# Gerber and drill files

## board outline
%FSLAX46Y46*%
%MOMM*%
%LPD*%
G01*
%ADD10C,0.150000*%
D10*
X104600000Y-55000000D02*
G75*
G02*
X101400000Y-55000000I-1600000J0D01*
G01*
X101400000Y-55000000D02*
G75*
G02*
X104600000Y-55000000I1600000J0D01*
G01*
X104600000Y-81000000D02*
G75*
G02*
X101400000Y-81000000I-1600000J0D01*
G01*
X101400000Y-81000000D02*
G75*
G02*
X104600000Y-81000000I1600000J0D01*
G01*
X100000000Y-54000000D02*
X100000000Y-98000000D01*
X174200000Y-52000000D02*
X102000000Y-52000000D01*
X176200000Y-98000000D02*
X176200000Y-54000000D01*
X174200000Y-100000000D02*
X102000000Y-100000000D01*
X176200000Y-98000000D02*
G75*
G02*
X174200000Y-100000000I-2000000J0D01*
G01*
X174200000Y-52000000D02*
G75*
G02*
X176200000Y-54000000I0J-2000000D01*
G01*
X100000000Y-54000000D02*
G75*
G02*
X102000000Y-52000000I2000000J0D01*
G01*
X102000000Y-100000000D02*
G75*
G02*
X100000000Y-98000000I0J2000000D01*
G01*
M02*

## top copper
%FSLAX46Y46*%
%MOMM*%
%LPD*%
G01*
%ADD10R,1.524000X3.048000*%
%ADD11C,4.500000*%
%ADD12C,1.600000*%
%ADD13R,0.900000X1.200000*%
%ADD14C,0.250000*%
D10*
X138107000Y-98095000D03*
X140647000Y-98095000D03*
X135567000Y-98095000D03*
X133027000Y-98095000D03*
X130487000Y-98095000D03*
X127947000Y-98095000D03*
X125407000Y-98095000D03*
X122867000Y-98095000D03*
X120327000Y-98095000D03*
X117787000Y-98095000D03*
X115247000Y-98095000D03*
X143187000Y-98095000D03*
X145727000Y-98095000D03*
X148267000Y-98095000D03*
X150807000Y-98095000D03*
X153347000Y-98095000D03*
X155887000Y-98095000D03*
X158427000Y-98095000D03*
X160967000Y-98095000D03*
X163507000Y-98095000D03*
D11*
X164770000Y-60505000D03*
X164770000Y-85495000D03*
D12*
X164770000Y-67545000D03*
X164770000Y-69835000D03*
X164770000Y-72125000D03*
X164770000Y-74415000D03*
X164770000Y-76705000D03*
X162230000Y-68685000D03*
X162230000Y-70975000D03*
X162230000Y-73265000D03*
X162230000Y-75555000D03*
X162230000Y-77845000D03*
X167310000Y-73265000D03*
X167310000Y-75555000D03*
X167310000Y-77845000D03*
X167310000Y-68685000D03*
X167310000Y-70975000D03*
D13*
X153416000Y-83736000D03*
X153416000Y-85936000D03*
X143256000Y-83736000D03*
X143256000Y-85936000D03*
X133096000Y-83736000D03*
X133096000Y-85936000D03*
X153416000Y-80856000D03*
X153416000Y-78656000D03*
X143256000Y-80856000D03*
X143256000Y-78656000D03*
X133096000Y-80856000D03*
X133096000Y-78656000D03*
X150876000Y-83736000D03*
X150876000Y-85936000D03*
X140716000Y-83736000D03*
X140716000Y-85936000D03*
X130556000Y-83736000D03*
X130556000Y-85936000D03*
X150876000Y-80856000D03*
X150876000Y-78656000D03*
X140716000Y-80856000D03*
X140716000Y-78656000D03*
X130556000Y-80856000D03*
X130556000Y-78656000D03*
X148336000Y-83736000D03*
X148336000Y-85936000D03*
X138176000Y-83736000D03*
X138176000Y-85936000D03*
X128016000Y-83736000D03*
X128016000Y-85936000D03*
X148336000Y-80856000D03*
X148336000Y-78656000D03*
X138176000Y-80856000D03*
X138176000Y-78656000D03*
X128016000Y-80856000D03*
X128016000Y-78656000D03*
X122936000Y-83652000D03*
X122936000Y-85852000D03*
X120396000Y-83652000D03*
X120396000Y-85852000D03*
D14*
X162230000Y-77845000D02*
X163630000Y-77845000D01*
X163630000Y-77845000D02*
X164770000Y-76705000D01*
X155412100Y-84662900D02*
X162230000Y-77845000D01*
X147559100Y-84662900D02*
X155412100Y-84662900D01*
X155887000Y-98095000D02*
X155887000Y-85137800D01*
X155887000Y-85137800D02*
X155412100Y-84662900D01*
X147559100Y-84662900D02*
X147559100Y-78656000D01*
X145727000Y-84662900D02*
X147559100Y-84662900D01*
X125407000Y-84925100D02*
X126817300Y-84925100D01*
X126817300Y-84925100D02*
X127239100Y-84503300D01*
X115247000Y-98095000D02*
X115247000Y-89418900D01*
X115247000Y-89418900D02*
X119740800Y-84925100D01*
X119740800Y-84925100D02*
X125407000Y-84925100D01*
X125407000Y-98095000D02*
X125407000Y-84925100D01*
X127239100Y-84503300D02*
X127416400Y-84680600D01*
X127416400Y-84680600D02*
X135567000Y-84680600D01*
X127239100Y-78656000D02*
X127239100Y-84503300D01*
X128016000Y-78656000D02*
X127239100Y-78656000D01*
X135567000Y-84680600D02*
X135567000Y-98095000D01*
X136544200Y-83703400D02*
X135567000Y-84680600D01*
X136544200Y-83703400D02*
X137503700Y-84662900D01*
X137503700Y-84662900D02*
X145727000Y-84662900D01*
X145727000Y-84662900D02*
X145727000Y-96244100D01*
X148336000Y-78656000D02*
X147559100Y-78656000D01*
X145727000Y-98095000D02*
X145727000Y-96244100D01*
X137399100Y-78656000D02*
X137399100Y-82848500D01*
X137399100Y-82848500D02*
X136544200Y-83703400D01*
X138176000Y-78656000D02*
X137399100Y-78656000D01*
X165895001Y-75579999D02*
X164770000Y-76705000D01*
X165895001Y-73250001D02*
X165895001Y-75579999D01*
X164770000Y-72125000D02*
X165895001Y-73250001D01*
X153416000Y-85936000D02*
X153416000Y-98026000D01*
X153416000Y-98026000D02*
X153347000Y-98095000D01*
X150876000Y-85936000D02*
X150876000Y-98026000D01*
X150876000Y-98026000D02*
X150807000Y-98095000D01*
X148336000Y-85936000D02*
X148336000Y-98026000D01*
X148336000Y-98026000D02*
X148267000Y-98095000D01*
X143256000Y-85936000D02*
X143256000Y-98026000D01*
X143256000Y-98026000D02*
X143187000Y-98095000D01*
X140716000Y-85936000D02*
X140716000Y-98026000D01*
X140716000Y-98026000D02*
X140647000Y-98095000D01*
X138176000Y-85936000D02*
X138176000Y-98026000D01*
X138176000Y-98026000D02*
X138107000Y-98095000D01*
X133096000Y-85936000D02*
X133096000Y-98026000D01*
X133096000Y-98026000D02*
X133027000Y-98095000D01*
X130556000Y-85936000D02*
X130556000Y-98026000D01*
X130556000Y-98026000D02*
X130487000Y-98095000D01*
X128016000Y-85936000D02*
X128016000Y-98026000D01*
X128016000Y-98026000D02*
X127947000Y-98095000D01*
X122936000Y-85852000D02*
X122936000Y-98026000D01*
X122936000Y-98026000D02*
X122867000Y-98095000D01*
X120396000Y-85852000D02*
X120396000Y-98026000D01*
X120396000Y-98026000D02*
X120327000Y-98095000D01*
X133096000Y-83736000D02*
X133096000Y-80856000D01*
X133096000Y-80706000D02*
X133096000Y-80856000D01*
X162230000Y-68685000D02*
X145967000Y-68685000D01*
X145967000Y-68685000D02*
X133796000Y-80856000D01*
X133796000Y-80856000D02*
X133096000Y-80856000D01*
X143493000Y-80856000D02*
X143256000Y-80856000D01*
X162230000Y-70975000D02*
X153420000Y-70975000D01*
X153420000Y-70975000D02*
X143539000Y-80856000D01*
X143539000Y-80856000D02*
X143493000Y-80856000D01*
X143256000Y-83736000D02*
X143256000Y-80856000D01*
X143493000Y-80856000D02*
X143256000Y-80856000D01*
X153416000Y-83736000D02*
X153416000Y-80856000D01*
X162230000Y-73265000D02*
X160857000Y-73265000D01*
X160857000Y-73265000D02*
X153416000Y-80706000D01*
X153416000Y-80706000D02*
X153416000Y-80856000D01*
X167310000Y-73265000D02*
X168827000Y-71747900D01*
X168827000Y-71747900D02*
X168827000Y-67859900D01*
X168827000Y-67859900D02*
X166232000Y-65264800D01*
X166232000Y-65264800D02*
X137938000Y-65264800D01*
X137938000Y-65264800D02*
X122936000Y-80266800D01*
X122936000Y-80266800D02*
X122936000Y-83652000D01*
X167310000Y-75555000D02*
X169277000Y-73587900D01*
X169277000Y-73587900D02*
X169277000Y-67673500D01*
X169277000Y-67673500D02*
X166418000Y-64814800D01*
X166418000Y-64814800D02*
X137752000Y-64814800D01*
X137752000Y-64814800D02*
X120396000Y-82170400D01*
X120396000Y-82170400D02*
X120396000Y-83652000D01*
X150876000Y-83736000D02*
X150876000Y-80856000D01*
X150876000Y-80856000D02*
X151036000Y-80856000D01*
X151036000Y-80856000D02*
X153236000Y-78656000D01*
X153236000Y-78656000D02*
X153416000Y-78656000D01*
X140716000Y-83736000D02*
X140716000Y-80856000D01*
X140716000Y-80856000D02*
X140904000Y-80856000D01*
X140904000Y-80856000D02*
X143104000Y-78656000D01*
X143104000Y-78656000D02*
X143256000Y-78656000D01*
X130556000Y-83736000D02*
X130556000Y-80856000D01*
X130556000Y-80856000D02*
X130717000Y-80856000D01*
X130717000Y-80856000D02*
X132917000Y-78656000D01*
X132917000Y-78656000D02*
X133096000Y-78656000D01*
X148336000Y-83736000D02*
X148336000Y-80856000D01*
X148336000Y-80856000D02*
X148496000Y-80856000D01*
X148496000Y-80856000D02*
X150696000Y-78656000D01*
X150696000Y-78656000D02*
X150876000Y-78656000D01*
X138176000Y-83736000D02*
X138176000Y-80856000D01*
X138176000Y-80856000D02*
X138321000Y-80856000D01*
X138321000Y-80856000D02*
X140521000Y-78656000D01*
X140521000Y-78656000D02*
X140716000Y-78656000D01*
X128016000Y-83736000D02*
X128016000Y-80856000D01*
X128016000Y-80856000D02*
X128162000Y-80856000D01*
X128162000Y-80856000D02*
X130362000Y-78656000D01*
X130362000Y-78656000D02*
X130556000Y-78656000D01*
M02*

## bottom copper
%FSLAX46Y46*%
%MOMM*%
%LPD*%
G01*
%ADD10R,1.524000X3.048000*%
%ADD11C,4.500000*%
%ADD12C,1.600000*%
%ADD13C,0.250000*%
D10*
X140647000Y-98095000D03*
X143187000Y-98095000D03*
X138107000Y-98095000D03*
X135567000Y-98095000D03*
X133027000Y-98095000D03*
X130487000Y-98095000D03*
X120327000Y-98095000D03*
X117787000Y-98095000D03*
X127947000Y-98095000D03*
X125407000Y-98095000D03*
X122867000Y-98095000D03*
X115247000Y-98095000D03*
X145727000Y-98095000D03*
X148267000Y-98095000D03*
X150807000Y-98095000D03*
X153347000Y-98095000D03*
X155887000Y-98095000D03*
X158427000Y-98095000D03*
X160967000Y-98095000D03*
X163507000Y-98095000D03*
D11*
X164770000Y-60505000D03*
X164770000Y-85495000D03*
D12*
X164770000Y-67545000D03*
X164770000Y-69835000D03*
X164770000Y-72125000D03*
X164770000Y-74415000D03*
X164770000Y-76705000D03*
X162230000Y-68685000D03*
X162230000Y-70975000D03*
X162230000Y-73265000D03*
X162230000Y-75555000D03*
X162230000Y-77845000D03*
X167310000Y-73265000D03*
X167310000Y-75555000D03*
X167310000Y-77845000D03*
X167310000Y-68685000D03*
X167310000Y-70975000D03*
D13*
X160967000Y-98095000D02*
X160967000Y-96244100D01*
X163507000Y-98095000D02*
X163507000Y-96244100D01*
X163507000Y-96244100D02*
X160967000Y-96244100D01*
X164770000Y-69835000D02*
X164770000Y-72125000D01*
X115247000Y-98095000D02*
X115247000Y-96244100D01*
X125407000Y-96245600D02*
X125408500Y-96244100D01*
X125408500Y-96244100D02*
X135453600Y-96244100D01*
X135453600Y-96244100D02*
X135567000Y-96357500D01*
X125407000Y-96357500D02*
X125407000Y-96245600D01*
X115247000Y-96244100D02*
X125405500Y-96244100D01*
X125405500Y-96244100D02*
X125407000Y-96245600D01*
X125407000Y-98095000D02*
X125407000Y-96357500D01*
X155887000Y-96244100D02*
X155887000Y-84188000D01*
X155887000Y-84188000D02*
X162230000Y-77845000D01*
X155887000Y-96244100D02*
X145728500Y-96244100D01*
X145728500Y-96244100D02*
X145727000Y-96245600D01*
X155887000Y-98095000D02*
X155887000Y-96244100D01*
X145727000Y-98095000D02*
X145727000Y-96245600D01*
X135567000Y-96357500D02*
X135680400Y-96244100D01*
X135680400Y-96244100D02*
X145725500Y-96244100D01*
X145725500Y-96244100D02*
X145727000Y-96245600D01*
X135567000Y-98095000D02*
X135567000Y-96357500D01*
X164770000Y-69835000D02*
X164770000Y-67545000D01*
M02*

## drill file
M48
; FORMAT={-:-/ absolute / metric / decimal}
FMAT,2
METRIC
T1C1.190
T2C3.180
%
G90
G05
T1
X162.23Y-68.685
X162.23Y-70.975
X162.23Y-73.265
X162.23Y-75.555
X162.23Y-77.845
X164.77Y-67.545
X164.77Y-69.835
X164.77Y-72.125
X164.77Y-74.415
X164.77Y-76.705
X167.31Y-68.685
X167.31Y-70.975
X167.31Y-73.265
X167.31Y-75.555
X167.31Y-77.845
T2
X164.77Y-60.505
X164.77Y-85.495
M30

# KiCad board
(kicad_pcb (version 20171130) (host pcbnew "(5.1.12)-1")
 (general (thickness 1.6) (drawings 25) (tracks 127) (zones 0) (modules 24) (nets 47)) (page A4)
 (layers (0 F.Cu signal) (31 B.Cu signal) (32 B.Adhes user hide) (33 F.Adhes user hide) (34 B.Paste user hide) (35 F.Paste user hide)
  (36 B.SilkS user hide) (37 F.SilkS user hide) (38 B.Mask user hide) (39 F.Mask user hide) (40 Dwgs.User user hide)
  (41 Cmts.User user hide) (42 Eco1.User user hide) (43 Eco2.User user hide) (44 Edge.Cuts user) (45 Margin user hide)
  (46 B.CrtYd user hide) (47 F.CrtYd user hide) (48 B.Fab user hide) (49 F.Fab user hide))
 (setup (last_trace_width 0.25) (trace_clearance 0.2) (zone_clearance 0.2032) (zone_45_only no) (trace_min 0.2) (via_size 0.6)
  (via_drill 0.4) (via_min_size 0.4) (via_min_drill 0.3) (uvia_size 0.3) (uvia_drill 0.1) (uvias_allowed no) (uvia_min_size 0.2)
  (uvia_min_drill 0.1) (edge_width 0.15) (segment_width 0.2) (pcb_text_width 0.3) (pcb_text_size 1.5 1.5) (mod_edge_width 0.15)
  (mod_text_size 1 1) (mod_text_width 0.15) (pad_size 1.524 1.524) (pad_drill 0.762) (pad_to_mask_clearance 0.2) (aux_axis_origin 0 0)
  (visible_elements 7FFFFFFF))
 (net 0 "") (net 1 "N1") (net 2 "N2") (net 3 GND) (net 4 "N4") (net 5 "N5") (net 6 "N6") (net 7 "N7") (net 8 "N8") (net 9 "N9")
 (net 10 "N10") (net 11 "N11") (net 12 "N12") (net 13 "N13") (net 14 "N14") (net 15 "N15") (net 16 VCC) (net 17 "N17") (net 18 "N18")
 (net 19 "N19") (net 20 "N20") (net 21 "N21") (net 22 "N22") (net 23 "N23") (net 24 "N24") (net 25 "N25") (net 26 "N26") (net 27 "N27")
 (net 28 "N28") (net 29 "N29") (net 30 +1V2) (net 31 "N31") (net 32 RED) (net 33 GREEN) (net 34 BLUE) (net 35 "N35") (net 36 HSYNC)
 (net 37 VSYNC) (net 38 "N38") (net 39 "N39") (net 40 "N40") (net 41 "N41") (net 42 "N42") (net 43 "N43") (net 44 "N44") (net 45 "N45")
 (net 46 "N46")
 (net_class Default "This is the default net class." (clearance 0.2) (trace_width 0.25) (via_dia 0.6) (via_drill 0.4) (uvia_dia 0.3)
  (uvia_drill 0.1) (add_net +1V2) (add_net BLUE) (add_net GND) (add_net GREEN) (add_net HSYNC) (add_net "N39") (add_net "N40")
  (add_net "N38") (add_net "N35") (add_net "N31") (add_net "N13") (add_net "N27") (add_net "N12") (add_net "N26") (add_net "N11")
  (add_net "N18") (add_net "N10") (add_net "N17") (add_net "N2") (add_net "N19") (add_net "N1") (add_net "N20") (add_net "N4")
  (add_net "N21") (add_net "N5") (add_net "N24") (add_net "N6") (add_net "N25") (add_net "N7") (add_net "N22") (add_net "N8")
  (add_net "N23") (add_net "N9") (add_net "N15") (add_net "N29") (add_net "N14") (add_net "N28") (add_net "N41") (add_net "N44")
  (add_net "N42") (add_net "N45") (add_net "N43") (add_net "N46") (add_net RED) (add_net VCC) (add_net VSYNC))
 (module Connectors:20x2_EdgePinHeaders (layer F.Cu) (at 139.377 100)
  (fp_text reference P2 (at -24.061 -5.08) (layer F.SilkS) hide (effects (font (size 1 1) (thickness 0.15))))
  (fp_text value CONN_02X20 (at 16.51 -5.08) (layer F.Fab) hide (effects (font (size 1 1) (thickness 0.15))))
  (pad 22 smd rect (at -1.27 -1.905) (size 1.524 3.048) (layers F.Cu F.Paste F.Mask) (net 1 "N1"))
  (pad 20 smd rect (at 1.27 -1.905) (size 1.524 3.048) (layers F.Cu F.Paste F.Mask) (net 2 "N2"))
  (pad 24 smd rect (at -3.81 -1.905) (size 1.524 3.048) (layers F.Cu F.Paste F.Mask) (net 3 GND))
  (pad 26 smd rect (at -6.35 -1.905) (size 1.524 3.048) (layers F.Cu F.Paste F.Mask) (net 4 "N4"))
  (pad 28 smd rect (at -8.89 -1.905) (size 1.524 3.048) (layers F.Cu F.Paste F.Mask) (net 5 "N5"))
  (pad 30 smd rect (at -11.43 -1.905) (size 1.524 3.048) (layers F.Cu F.Paste F.Mask) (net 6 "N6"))
  (pad 32 smd rect (at -13.97 -1.905) (size 1.524 3.048) (layers F.Cu F.Paste F.Mask) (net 3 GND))
  (pad 34 smd rect (at -16.51 -1.905) (size 1.524 3.048) (layers F.Cu F.Paste F.Mask) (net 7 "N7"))
  (pad 36 smd rect (at -19.05 -1.905) (size 1.524 3.048) (layers F.Cu F.Paste F.Mask) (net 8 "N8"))
  (pad 38 smd rect (at -21.59 -1.905) (size 1.524 3.048) (layers F.Cu F.Paste F.Mask) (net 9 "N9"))
  (pad 40 smd rect (at -24.13 -1.905) (size 1.524 3.048) (layers F.Cu F.Paste F.Mask) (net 3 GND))
  (pad 18 smd rect (at 3.81 -1.905) (size 1.524 3.048) (layers F.Cu F.Paste F.Mask) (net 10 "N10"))
  (pad 16 smd rect (at 6.35 -1.905) (size 1.524 3.048) (layers F.Cu F.Paste F.Mask) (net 3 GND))
  (pad 14 smd rect (at 8.89 -1.905) (size 1.524 3.048) (layers F.Cu F.Paste F.Mask) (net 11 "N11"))
  (pad 12 smd rect (at 11.43 -1.905) (size 1.524 3.048) (layers F.Cu F.Paste F.Mask) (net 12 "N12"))
  (pad 10 smd rect (at 13.97 -1.905) (size 1.524 3.048) (layers F.Cu F.Paste F.Mask) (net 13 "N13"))
  (pad 8 smd rect (at 16.51 -1.905) (size 1.524 3.048) (layers F.Cu F.Paste F.Mask) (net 3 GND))
  (pad 6 smd rect (at 19.05 -1.905) (size 1.524 3.048) (layers F.Cu F.Paste F.Mask) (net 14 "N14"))
  (pad 4 smd rect (at 21.59 -1.905) (size 1.524 3.048) (layers F.Cu F.Paste F.Mask) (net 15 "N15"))
  (pad 2 smd rect (at 24.13 -1.905) (size 1.524 3.048) (layers F.Cu F.Paste F.Mask) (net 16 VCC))
  (pad 19 smd rect (at 1.27 -1.905) (size 1.524 3.048) (layers B.Cu B.Paste B.Mask) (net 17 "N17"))
  (pad 17 smd rect (at 3.81 -1.905) (size 1.524 3.048) (layers B.Cu B.Paste B.Mask) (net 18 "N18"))
  (pad 21 smd rect (at -1.27 -1.905) (size 1.524 3.048) (layers B.Cu B.Paste B.Mask) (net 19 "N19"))
  (pad 23 smd rect (at -3.81 -1.905) (size 1.524 3.048) (layers B.Cu B.Paste B.Mask) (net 3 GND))
  (pad 25 smd rect (at -6.35 -1.905) (size 1.524 3.048) (layers B.Cu B.Paste B.Mask) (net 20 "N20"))
  (pad 27 smd rect (at -8.89 -1.905) (size 1.524 3.048) (layers B.Cu B.Paste B.Mask) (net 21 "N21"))
  (pad 35 smd rect (at -19.05 -1.905) (size 1.524 3.048) (layers B.Cu B.Paste B.Mask) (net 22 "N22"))
  (pad 37 smd rect (at -21.59 -1.905) (size 1.524 3.048) (layers B.Cu B.Paste B.Mask) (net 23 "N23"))
  (pad 29 smd rect (at -11.43 -1.905) (size 1.524 3.048) (layers B.Cu B.Paste B.Mask) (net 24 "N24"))
  (pad 31 smd rect (at -13.97 -1.905) (size 1.524 3.048) (layers B.Cu B.Paste B.Mask) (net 3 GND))
  (pad 33 smd rect (at -16.51 -1.905) (size 1.524 3.048) (layers B.Cu B.Paste B.Mask) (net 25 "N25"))
  (pad 39 smd rect (at -24.13 -1.905) (size 1.524 3.048) (layers B.Cu B.Paste B.Mask) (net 3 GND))
  (pad 15 smd rect (at 6.35 -1.905) (size 1.524 3.048) (layers B.Cu B.Paste B.Mask) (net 3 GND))
  (pad 13 smd rect (at 8.89 -1.905) (size 1.524 3.048) (layers B.Cu B.Paste B.Mask) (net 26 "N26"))
  (pad 11 smd rect (at 11.43 -1.905) (size 1.524 3.048) (layers B.Cu B.Paste B.Mask) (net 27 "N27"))
  (pad 9 smd rect (at 13.97 -1.905) (size 1.524 3.048) (layers B.Cu B.Paste B.Mask) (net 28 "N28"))
  (pad 7 smd rect (at 16.51 -1.905) (size 1.524 3.048) (layers B.Cu B.Paste B.Mask) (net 3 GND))
  (pad 5 smd rect (at 19.05 -1.905) (size 1.524 3.048) (layers B.Cu B.Paste B.Mask) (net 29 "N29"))
  (pad 3 smd rect (at 21.59 -1.905) (size 1.524 3.048) (layers B.Cu B.Paste B.Mask) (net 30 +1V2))
  (pad 1 smd rect (at 24.13 -1.905) (size 1.524 3.048) (layers B.Cu B.Paste B.Mask) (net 30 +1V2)))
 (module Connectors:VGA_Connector (layer F.Cu) (at 176.2 73)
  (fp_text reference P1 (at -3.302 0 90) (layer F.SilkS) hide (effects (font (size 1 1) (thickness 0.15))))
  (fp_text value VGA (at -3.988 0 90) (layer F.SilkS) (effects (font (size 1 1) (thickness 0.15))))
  (pad "" thru_hole circle (at -11.43 -12.495) (size 4.5 4.5) (drill 3.18) (layers *.Cu *.Mask F.SilkS))
  (pad "" thru_hole circle (at -11.43 12.495) (size 4.5 4.5) (drill 3.18) (layers *.Cu *.Mask F.SilkS))
  (pad 6 thru_hole circle (at -11.43 -5.455) (size 1.6 1.6) (drill 1.19) (layers *.Cu *.Mask F.SilkS) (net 3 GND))
  (pad 7 thru_hole circle (at -11.43 -3.165) (size 1.6 1.6) (drill 1.19) (layers *.Cu *.Mask F.SilkS) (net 3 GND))
  (pad 8 thru_hole circle (at -11.43 -0.875) (size 1.6 1.6) (drill 1.19) (layers *.Cu *.Mask F.SilkS) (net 3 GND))
  (pad 9 thru_hole circle (at -11.43 1.415) (size 1.6 1.6) (drill 1.19) (layers *.Cu *.Mask F.SilkS) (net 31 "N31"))
  (pad 10 thru_hole circle (at -11.43 3.705) (size 1.6 1.6) (drill 1.19) (layers *.Cu *.Mask F.SilkS) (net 3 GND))
  (pad 1 thru_hole circle (at -13.97 -4.315) (size 1.6 1.6) (drill 1.19) (layers *.Cu *.Mask F.SilkS) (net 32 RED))
  (pad 2 thru_hole circle (at -13.97 -2.025) (size 1.6 1.6) (drill 1.19) (layers *.Cu *.Mask F.SilkS) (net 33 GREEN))
  (pad 3 thru_hole circle (at -13.97 0.265) (size 1.6 1.6) (drill 1.19) (layers *.Cu *.Mask F.SilkS) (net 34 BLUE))
  (pad 4 thru_hole circle (at -13.97 2.555) (size 1.6 1.6) (drill 1.19) (layers *.Cu *.Mask F.SilkS) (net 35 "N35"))
  (pad 5 thru_hole circle (at -13.97 4.845) (size 1.6 1.6) (drill 1.19) (layers *.Cu *.Mask F.SilkS) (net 3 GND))
  (pad 13 thru_hole circle (at -8.89 0.265) (size 1.6 1.6) (drill 1.19) (layers *.Cu *.Mask F.SilkS) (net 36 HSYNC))
  (pad 14 thru_hole circle (at -8.89 2.555) (size 1.6 1.6) (drill 1.19) (layers *.Cu *.Mask F.SilkS) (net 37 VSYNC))
  (pad 15 thru_hole circle (at -8.89 4.845) (size 1.6 1.6) (drill 1.19) (layers *.Cu *.Mask F.SilkS) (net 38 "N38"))
  (pad 11 thru_hole circle (at -8.89 -4.315) (size 1.6 1.6) (drill 1.19) (layers *.Cu *.Mask F.SilkS) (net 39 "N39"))
  (pad 12 thru_hole circle (at -8.89 -2.025) (size 1.6 1.6) (drill 1.19) (layers *.Cu *.Mask F.SilkS) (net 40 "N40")))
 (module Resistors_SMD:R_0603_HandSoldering (layer F.Cu) (at 153.416 84.836 270)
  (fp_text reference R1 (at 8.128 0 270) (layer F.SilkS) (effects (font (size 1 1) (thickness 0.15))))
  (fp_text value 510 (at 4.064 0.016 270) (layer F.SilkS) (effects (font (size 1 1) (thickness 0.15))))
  (pad 1 smd rect (at -1.1 0 270) (size 1.2 0.9) (layers F.Cu F.Paste F.Mask) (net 34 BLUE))
  (pad 2 smd rect (at 1.1 0 270) (size 1.2 0.9) (layers F.Cu F.Paste F.Mask) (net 13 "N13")))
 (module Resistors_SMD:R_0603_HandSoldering (layer F.Cu) (at 143.256 84.836 270)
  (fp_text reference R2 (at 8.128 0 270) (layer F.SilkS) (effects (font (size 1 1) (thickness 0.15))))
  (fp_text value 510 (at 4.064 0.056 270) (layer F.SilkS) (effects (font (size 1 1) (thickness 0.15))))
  (pad 1 smd rect (at -1.1 0 270) (size 1.2 0.9) (layers F.Cu F.Paste F.Mask) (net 33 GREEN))
  (pad 2 smd rect (at 1.1 0 270) (size 1.2 0.9) (layers F.Cu F.Paste F.Mask) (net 10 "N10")))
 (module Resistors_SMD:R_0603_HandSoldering (layer F.Cu) (at 133.096 84.836 270)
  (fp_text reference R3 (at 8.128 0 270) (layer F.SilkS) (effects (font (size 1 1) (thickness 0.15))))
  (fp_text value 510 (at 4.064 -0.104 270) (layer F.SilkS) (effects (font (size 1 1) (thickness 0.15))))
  (pad 1 smd rect (at -1.1 0 270) (size 1.2 0.9) (layers F.Cu F.Paste F.Mask) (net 32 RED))
  (pad 2 smd rect (at 1.1 0 270) (size 1.2 0.9) (layers F.Cu F.Paste F.Mask) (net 4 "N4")))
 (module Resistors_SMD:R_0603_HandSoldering (layer F.Cu) (at 153.416 79.756 90)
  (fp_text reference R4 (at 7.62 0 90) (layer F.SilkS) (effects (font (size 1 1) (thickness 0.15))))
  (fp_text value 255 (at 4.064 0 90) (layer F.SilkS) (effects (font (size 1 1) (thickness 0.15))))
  (pad 1 smd rect (at -1.1 0 90) (size 1.2 0.9) (layers F.Cu F.Paste F.Mask) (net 34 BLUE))
  (pad 2 smd rect (at 1.1 0 90) (size 1.2 0.9) (layers F.Cu F.Paste F.Mask) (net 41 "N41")))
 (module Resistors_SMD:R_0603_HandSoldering (layer F.Cu) (at 143.256 79.756 90)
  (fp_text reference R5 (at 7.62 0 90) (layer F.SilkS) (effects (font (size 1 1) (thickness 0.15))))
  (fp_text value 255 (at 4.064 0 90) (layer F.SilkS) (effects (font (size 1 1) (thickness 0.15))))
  (pad 1 smd rect (at -1.1 0 90) (size 1.2 0.9) (layers F.Cu F.Paste F.Mask) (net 33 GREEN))
  (pad 2 smd rect (at 1.1 0 90) (size 1.2 0.9) (layers F.Cu F.Paste F.Mask) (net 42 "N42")))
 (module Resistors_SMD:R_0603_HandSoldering (layer F.Cu) (at 133.096 79.756 90)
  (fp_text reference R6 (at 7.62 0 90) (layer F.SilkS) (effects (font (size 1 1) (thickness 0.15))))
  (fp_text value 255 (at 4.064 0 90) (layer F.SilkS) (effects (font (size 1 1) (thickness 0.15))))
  (pad 1 smd rect (at -1.1 0 90) (size 1.2 0.9) (layers F.Cu F.Paste F.Mask) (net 32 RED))
  (pad 2 smd rect (at 1.1 0 90) (size 1.2 0.9) (layers F.Cu F.Paste F.Mask) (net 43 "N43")))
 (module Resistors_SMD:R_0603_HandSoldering (layer F.Cu) (at 150.876 84.836 270)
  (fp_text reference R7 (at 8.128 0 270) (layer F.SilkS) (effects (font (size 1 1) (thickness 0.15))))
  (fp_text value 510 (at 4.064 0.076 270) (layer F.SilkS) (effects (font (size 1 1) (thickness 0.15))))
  (pad 1 smd rect (at -1.1 0 270) (size 1.2 0.9) (layers F.Cu F.Paste F.Mask) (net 41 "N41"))
  (pad 2 smd rect (at 1.1 0 270) (size 1.2 0.9) (layers F.Cu F.Paste F.Mask) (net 12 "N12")))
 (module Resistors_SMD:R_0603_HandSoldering (layer F.Cu) (at 140.716 84.836 270)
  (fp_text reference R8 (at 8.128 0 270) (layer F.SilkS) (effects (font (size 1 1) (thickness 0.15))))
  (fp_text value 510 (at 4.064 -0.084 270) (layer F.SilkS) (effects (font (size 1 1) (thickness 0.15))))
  (pad 1 smd rect (at -1.1 0 270) (size 1.2 0.9) (layers F.Cu F.Paste F.Mask) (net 42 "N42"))
  (pad 2 smd rect (at 1.1 0 270) (size 1.2 0.9) (layers F.Cu F.Paste F.Mask) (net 2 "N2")))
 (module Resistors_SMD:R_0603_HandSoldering (layer F.Cu) (at 130.556 84.836 270)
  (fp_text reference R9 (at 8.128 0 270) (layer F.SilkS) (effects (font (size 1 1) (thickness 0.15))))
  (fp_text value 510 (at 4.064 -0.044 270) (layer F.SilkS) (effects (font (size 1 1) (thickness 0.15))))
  (pad 1 smd rect (at -1.1 0 270) (size 1.2 0.9) (layers F.Cu F.Paste F.Mask) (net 43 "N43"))
  (pad 2 smd rect (at 1.1 0 270) (size 1.2 0.9) (layers F.Cu F.Paste F.Mask) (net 5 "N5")))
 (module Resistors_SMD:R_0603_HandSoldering (layer F.Cu) (at 150.876 79.756 90)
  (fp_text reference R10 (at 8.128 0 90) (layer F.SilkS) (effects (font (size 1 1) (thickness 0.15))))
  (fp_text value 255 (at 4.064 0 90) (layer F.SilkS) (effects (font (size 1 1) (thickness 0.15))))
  (pad 1 smd rect (at -1.1 0 90) (size 1.2 0.9) (layers F.Cu F.Paste F.Mask) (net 41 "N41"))
  (pad 2 smd rect (at 1.1 0 90) (size 1.2 0.9) (layers F.Cu F.Paste F.Mask) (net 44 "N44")))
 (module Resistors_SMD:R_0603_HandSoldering (layer F.Cu) (at 140.716 79.756 90)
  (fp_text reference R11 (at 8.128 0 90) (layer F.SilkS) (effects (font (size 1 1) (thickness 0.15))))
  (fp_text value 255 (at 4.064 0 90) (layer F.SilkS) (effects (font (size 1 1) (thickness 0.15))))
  (pad 1 smd rect (at -1.1 0 90) (size 1.2 0.9) (layers F.Cu F.Paste F.Mask) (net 42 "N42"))
  (pad 2 smd rect (at 1.1 0 90) (size 1.2 0.9) (layers F.Cu F.Paste F.Mask) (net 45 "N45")))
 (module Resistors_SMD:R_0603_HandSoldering (layer F.Cu) (at 130.556 79.756 90)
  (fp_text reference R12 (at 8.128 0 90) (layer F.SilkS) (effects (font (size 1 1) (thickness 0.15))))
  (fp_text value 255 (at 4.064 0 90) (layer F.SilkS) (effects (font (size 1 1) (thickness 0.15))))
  (pad 1 smd rect (at -1.1 0 90) (size 1.2 0.9) (layers F.Cu F.Paste F.Mask) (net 43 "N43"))
  (pad 2 smd rect (at 1.1 0 90) (size 1.2 0.9) (layers F.Cu F.Paste F.Mask) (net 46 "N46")))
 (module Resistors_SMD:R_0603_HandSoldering (layer F.Cu) (at 148.336 84.836 270)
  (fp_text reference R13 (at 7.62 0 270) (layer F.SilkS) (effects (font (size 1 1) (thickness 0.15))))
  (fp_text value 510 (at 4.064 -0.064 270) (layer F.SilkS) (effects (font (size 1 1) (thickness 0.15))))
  (pad 1 smd rect (at -1.1 0 270) (size 1.2 0.9) (layers F.Cu F.Paste F.Mask) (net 44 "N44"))
  (pad 2 smd rect (at 1.1 0 270) (size 1.2 0.9) (layers F.Cu F.Paste F.Mask) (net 11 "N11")))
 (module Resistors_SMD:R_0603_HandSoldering (layer F.Cu) (at 138.176 84.836 270)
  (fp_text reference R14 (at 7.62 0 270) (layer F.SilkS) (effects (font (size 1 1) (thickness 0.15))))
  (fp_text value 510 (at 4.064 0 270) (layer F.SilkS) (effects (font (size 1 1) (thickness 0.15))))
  (pad 1 smd rect (at -1.1 0 270) (size 1.2 0.9) (layers F.Cu F.Paste F.Mask) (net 45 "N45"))
  (pad 2 smd rect (at 1.1 0 270) (size 1.2 0.9) (layers F.Cu F.Paste F.Mask) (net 1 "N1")))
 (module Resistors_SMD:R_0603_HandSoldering (layer F.Cu) (at 128.016 84.836 270)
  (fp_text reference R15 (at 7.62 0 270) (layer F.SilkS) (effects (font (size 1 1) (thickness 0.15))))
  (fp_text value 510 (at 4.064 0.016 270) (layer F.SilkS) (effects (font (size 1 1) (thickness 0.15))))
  (pad 1 smd rect (at -1.1 0 270) (size 1.2 0.9) (layers F.Cu F.Paste F.Mask) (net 46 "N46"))
  (pad 2 smd rect (at 1.1 0 270) (size 1.2 0.9) (layers F.Cu F.Paste F.Mask) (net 6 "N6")))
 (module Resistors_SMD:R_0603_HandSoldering (layer F.Cu) (at 148.336 79.756 90)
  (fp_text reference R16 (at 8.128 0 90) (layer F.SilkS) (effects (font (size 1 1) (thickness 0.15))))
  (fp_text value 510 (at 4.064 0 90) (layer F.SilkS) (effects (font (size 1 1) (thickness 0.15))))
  (pad 1 smd rect (at -1.1 0 90) (size 1.2 0.9) (layers F.Cu F.Paste F.Mask) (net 44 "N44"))
  (pad 2 smd rect (at 1.1 0 90) (size 1.2 0.9) (layers F.Cu F.Paste F.Mask) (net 3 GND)))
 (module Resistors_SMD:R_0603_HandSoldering (layer F.Cu) (at 138.176 79.756 90)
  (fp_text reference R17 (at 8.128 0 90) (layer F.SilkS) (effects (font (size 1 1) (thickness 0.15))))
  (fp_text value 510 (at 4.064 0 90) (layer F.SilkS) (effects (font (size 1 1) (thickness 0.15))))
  (pad 1 smd rect (at -1.1 0 90) (size 1.2 0.9) (layers F.Cu F.Paste F.Mask) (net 45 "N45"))
  (pad 2 smd rect (at 1.1 0 90) (size 1.2 0.9) (layers F.Cu F.Paste F.Mask) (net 3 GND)))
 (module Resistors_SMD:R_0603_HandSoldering (layer F.Cu) (at 128.016 79.756 90)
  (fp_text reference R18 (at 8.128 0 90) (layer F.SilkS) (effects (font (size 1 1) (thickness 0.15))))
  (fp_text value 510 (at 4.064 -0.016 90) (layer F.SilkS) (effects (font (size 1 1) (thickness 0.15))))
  (pad 1 smd rect (at -1.1 0 90) (size 1.2 0.9) (layers F.Cu F.Paste F.Mask) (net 46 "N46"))
  (pad 2 smd rect (at 1.1 0 90) (size 1.2 0.9) (layers F.Cu F.Paste F.Mask) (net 3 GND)))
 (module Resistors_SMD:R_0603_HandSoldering (layer F.Cu) (at 122.936 84.752 270)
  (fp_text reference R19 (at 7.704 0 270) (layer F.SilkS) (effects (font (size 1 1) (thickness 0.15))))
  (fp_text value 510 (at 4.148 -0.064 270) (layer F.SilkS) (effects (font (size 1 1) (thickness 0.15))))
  (pad 1 smd rect (at -1.1 0 270) (size 1.2 0.9) (layers F.Cu F.Paste F.Mask) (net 36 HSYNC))
  (pad 2 smd rect (at 1.1 0 270) (size 1.2 0.9) (layers F.Cu F.Paste F.Mask) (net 7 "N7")))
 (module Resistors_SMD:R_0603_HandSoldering (layer F.Cu) (at 120.396 84.752 270)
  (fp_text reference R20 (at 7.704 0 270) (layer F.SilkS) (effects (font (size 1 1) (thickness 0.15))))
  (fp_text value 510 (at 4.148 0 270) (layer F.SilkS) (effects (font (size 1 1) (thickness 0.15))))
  (pad 1 smd rect (at -1.1 0 270) (size 1.2 0.9) (layers F.Cu F.Paste F.Mask) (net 37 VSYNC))
  (pad 2 smd rect (at 1.1 0 270) (size 1.2 0.9) (layers F.Cu F.Paste F.Mask) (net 8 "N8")))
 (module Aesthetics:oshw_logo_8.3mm (layer B.Cu) (at 157.988 90.424 180)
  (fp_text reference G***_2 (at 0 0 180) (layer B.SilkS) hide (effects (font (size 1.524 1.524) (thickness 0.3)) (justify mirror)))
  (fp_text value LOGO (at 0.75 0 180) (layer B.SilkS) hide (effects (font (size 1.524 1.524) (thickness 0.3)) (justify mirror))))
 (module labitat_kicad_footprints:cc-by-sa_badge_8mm (layer B.Cu) (at 124.968 90.424 180)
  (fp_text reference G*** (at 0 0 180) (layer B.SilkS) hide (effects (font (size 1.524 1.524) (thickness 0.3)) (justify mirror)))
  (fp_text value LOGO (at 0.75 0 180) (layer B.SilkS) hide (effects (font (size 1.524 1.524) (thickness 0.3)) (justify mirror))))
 (gr_circle (center 103 55) (end 101.4 55) (layer Edge.Cuts) (width 0.15))
 (gr_circle (center 103 81) (end 101.4 81) (layer Edge.Cuts) (width 0.15))
 (gr_line (start 100 54) (end 100 98) (layer Edge.Cuts) (width 0.15))
 (gr_line (start 174.2 52) (end 102 52) (layer Edge.Cuts) (width 0.15))
 (gr_line (start 176.2 98) (end 176.2 54) (layer Edge.Cuts) (width 0.15))
 (gr_line (start 174.2 100) (end 102 100) (layer Edge.Cuts) (width 0.15))
 (gr_arc (start 174.2 98) (end 176.2 98) (angle 90) (layer Edge.Cuts) (width 0.15))
 (gr_arc (start 174.2 54) (end 174.2 52) (angle 90) (layer Edge.Cuts) (width 0.15))
 (gr_arc (start 102 54) (end 100 54) (angle 90) (layer Edge.Cuts) (width 0.15))
 (gr_arc (start 102 98) (end 102 100) (angle 90) (layer Edge.Cuts) (width 0.15))
 (segment (start 160.967 98.095) (end 160.967 96.2441) (width 0.25) (layer B.Cu) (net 30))
 (segment (start 163.507 98.095) (end 163.507 96.2441) (width 0.25) (layer B.Cu) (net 30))
 (segment (start 163.507 96.2441) (end 160.967 96.2441) (width 0.25) (layer B.Cu) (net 30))
 (segment (start 162.23 77.845) (end 163.63 77.845) (width 0.25) (layer F.Cu) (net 3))
 (segment (start 163.63 77.845) (end 164.77 76.705) (width 0.25) (layer F.Cu) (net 3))
 (segment (start 155.4121 84.6629) (end 162.23 77.845) (width 0.25) (layer F.Cu) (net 3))
 (segment (start 147.5591 84.6629) (end 155.4121 84.6629) (width 0.25) (layer F.Cu) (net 3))
 (segment (start 155.887 98.095) (end 155.887 85.1378) (width 0.25) (layer F.Cu) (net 3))
 (segment (start 155.887 85.1378) (end 155.4121 84.6629) (width 0.25) (layer F.Cu) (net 3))
 (segment (start 147.5591 84.6629) (end 147.5591 78.656) (width 0.25) (layer F.Cu) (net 3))
 (segment (start 145.727 84.6629) (end 147.5591 84.6629) (width 0.25) (layer F.Cu) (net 3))
 (segment (start 164.77 69.835) (end 164.77 72.125) (width 0.25) (layer B.Cu) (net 3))
 (segment (start 125.407 84.9251) (end 126.8173 84.9251) (width 0.25) (layer F.Cu) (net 3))
 (segment (start 126.8173 84.9251) (end 127.2391 84.5033) (width 0.25) (layer F.Cu) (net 3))
 (segment (start 115.247 98.095) (end 115.247 89.4189) (width 0.25) (layer F.Cu) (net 3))
 (segment (start 115.247 89.4189) (end 119.7408 84.9251) (width 0.25) (layer F.Cu) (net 3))
 (segment (start 119.7408 84.9251) (end 125.407 84.9251) (width 0.25) (layer F.Cu) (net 3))
 (segment (start 125.407 98.095) (end 125.407 84.9251) (width 0.25) (layer F.Cu) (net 3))
 (segment (start 127.2391 84.5033) (end 127.4164 84.6806) (width 0.25) (layer F.Cu) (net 3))
 (segment (start 127.4164 84.6806) (end 135.567 84.6806) (width 0.25) (layer F.Cu) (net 3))
 (segment (start 127.2391 78.656) (end 127.2391 84.5033) (width 0.25) (layer F.Cu) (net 3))
 (segment (start 128.016 78.656) (end 127.2391 78.656) (width 0.25) (layer F.Cu) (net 3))
 (segment (start 135.567 84.6806) (end 135.567 98.095) (width 0.25) (layer F.Cu) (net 3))
 (segment (start 136.5442 83.7034) (end 135.567 84.6806) (width 0.25) (layer F.Cu) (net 3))
 (segment (start 115.247 98.095) (end 115.247 96.2441) (width 0.25) (layer B.Cu) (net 3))
 (segment (start 125.407 96.2456) (end 125.4085 96.2441) (width 0.25) (layer B.Cu) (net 3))
 (segment (start 125.4085 96.2441) (end 135.4536 96.2441) (width 0.25) (layer B.Cu) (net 3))
 (segment (start 135.4536 96.2441) (end 135.567 96.3575) (width 0.25) (layer B.Cu) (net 3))
 (segment (start 125.407 96.3575) (end 125.407 96.2456) (width 0.25) (layer B.Cu) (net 3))
 (segment (start 115.247 96.2441) (end 125.4055 96.2441) (width 0.25) (layer B.Cu) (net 3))
 (segment (start 125.4055 96.2441) (end 125.407 96.2456) (width 0.25) (layer B.Cu) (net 3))
 (segment (start 125.407 98.095) (end 125.407 96.3575) (width 0.25) (layer B.Cu) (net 3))
 (segment (start 155.887 96.2441) (end 155.887 84.188) (width 0.25) (layer B.Cu) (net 3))
 (segment (start 155.887 84.188) (end 162.23 77.845) (width 0.25) (layer B.Cu) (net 3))
 (segment (start 155.887 96.2441) (end 145.7285 96.2441) (width 0.25) (layer B.Cu) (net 3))
 (segment (start 145.7285 96.2441) (end 145.727 96.2456) (width 0.25) (layer B.Cu) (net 3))
 (segment (start 155.887 98.095) (end 155.887 96.2441) (width 0.25) (layer B.Cu) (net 3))
 (segment (start 136.5442 83.7034) (end 137.5037 84.6629) (width 0.25) (layer F.Cu) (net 3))
 (segment (start 137.5037 84.6629) (end 145.727 84.6629) (width 0.25) (layer F.Cu) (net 3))
 (segment (start 145.727 84.6629) (end 145.727 96.2441) (width 0.25) (layer F.Cu) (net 3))
 (segment (start 148.336 78.656) (end 147.5591 78.656) (width 0.25) (layer F.Cu) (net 3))
 (segment (start 145.727 98.095) (end 145.727 96.2441) (width 0.25) (layer F.Cu) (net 3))
 (segment (start 145.727 98.095) (end 145.727 96.2456) (width 0.25) (layer B.Cu) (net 3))
 (segment (start 135.567 96.3575) (end 135.6804 96.2441) (width 0.25) (layer B.Cu) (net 3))
 (segment (start 135.6804 96.2441) (end 145.7255 96.2441) (width 0.25) (layer B.Cu) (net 3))
 (segment (start 145.7255 96.2441) (end 145.727 96.2456) (width 0.25) (layer B.Cu) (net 3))
 (segment (start 135.567 98.095) (end 135.567 96.3575) (width 0.25) (layer B.Cu) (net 3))
 (segment (start 137.3991 78.656) (end 137.3991 82.8485) (width 0.25) (layer F.Cu) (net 3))
 (segment (start 137.3991 82.8485) (end 136.5442 83.7034) (width 0.25) (layer F.Cu) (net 3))
 (segment (start 138.176 78.656) (end 137.3991 78.656) (width 0.25) (layer F.Cu) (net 3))
 (segment (start 164.77 69.835) (end 164.77 67.545) (width 0.25) (layer B.Cu) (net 3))
 (segment (start 165.895001 75.579999) (end 164.77 76.705) (width 0.25) (layer F.Cu) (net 3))
 (segment (start 165.895001 73.250001) (end 165.895001 75.579999) (width 0.25) (layer F.Cu) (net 3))
 (segment (start 164.77 72.125) (end 165.895001 73.250001) (width 0.25) (layer F.Cu) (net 3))
 (segment (start 153.416 85.936) (end 153.416 98.026) (width 0.25) (layer F.Cu) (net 13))
 (segment (start 153.416 98.026) (end 153.347 98.095) (width 0.25) (layer F.Cu) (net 13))
 (segment (start 150.876 85.936) (end 150.876 98.026) (width 0.25) (layer F.Cu) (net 12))
 (segment (start 150.876 98.026) (end 150.807 98.095) (width 0.25) (layer F.Cu) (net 12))
 (segment (start 148.336 85.936) (end 148.336 98.026) (width 0.25) (layer F.Cu) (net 11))
 (segment (start 148.336 98.026) (end 148.267 98.095) (width 0.25) (layer F.Cu) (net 11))
 (segment (start 143.256 85.936) (end 143.256 98.026) (width 0.25) (layer F.Cu) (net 10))
 (segment (start 143.256 98.026) (end 143.187 98.095) (width 0.25) (layer F.Cu) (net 10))
 (segment (start 140.716 85.936) (end 140.716 98.026) (width 0.25) (layer F.Cu) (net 2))
 (segment (start 140.716 98.026) (end 140.647 98.095) (width 0.25) (layer F.Cu) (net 2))
 (segment (start 138.176 85.936) (end 138.176 98.026) (width 0.25) (layer F.Cu) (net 1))
 (segment (start 138.176 98.026) (end 138.107 98.095) (width 0.25) (layer F.Cu) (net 1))
 (segment (start 133.096 85.936) (end 133.096 98.026) (width 0.25) (layer F.Cu) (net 4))
 (segment (start 133.096 98.026) (end 133.027 98.095) (width 0.25) (layer F.Cu) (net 4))
 (segment (start 130.556 85.936) (end 130.556 98.026) (width 0.25) (layer F.Cu) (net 5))
 (segment (start 130.556 98.026) (end 130.487 98.095) (width 0.25) (layer F.Cu) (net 5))
 (segment (start 128.016 85.936) (end 128.016 98.026) (width 0.25) (layer F.Cu) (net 6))
 (segment (start 128.016 98.026) (end 127.947 98.095) (width 0.25) (layer F.Cu) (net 6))
 (segment (start 122.936 85.852) (end 122.936 98.026) (width 0.25) (layer F.Cu) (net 7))
 (segment (start 122.936 98.026) (end 122.867 98.095) (width 0.25) (layer F.Cu) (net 7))
 (segment (start 120.396 85.852) (end 120.396 98.026) (width 0.25) (layer F.Cu) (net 8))
 (segment (start 120.396 98.026) (end 120.327 98.095) (width 0.25) (layer F.Cu) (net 8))
 (segment (start 133.096 83.736) (end 133.096 80.856) (width 0.25) (layer F.Cu) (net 32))
 (segment (start 133.096 80.706) (end 133.096 80.856) (width 0.25) (layer F.Cu) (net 32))
 (segment (start 162.23 68.685) (end 145.967 68.685) (width 0.25) (layer F.Cu) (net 32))
 (segment (start 145.967 68.685) (end 133.796 80.856) (width 0.25) (layer F.Cu) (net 32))
 (segment (start 133.796 80.856) (end 133.096 80.856) (width 0.25) (layer F.Cu) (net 32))
 (segment (start 143.493 80.856) (end 143.256 80.856) (width 0.25) (layer F.Cu) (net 33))
 (segment (start 162.23 70.975) (end 153.42 70.975) (width 0.25) (layer F.Cu) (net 33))
 (segment (start 153.42 70.975) (end 143.539 80.856) (width 0.25) (layer F.Cu) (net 33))
 (segment (start 143.539 80.856) (end 143.493 80.856) (width 0.25) (layer F.Cu) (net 33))
 (segment (start 143.256 83.736) (end 143.256 80.856) (width 0.25) (layer F.Cu) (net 33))
 (segment (start 143.493 80.856) (end 143.256 80.856) (width 0.25) (layer F.Cu) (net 33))
 (segment (start 153.416 83.736) (end 153.416 80.856) (width 0.25) (layer F.Cu) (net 34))
 (segment (start 162.23 73.265) (end 160.857 73.265) (width 0.25) (layer F.Cu) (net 34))
 (segment (start 160.857 73.265) (end 153.416 80.706) (width 0.25) (layer F.Cu) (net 34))
 (segment (start 153.416 80.706) (end 153.416 80.856) (width 0.25) (layer F.Cu) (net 34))
 (segment (start 167.31 73.265) (end 168.827 71.7479) (width 0.25) (layer F.Cu) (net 36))
 (segment (start 168.827 71.7479) (end 168.827 67.8599) (width 0.25) (layer F.Cu) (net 36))
 (segment (start 168.827 67.8599) (end 166.232 65.2648) (width 0.25) (layer F.Cu) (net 36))
 (segment (start 166.232 65.2648) (end 137.938 65.2648) (width 0.25) (layer F.Cu) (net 36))
 (segment (start 137.938 65.2648) (end 122.936 80.2668) (width 0.25) (layer F.Cu) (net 36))
 (segment (start 122.936 80.2668) (end 122.936 83.652) (width 0.25) (layer F.Cu) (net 36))
 (segment (start 167.31 75.555) (end 169.277 73.5879) (width 0.25) (layer F.Cu) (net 37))
 (segment (start 169.277 73.5879) (end 169.277 67.6735) (width 0.25) (layer F.Cu) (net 37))
 (segment (start 169.277 67.6735) (end 166.418 64.8148) (width 0.25) (layer F.Cu) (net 37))
 (segment (start 166.418 64.8148) (end 137.752 64.8148) (width 0.25) (layer F.Cu) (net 37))
 (segment (start 137.752 64.8148) (end 120.396 82.1704) (width 0.25) (layer F.Cu) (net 37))
 (segment (start 120.396 82.1704) (end 120.396 83.652) (width 0.25) (layer F.Cu) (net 37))
 (segment (start 150.876 83.736) (end 150.876 80.856) (width 0.25) (layer F.Cu) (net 41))
 (segment (start 150.876 80.856) (end 151.036 80.856) (width 0.25) (layer F.Cu) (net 41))
 (segment (start 151.036 80.856) (end 153.236 78.656) (width 0.25) (layer F.Cu) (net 41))
 (segment (start 153.236 78.656) (end 153.416 78.656) (width 0.25) (layer F.Cu) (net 41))
 (segment (start 140.716 83.736) (end 140.716 80.856) (width 0.25) (layer F.Cu) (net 42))
 (segment (start 140.716 80.856) (end 140.904 80.856) (width 0.25) (layer F.Cu) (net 42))
 (segment (start 140.904 80.856) (end 143.104 78.656) (width 0.25) (layer F.Cu) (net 42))
 (segment (start 143.104 78.656) (end 143.256 78.656) (width 0.25) (layer F.Cu) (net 42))
 (segment (start 130.556 83.736) (end 130.556 80.856) (width 0.25) (layer F.Cu) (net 43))
 (segment (start 130.556 80.856) (end 130.717 80.856) (width 0.25) (layer F.Cu) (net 43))
 (segment (start 130.717 80.856) (end 132.917 78.656) (width 0.25) (layer F.Cu) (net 43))
 (segment (start 132.917 78.656) (end 133.096 78.656) (width 0.25) (layer F.Cu) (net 43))
 (segment (start 148.336 83.736) (end 148.336 80.856) (width 0.25) (layer F.Cu) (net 44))
 (segment (start 148.336 80.856) (end 148.496 80.856) (width 0.25) (layer F.Cu) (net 44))
 (segment (start 148.496 80.856) (end 150.696 78.656) (width 0.25) (layer F.Cu) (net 44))
 (segment (start 150.696 78.656) (end 150.876 78.656) (width 0.25) (layer F.Cu) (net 44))
 (segment (start 138.176 83.736) (end 138.176 80.856) (width 0.25) (layer F.Cu) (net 45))
 (segment (start 138.176 80.856) (end 138.321 80.856) (width 0.25) (layer F.Cu) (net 45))
 (segment (start 138.321 80.856) (end 140.521 78.656) (width 0.25) (layer F.Cu) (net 45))
 (segment (start 140.521 78.656) (end 140.716 78.656) (width 0.25) (layer F.Cu) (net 45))
 (segment (start 128.016 83.736) (end 128.016 80.856) (width 0.25) (layer F.Cu) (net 46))
 (segment (start 128.016 80.856) (end 128.162 80.856) (width 0.25) (layer F.Cu) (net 46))
 (segment (start 128.162 80.856) (end 130.362 78.656) (width 0.25) (layer F.Cu) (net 46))
 (segment (start 130.362 78.656) (end 130.556 78.656) (width 0.25) (layer F.Cu) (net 46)))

